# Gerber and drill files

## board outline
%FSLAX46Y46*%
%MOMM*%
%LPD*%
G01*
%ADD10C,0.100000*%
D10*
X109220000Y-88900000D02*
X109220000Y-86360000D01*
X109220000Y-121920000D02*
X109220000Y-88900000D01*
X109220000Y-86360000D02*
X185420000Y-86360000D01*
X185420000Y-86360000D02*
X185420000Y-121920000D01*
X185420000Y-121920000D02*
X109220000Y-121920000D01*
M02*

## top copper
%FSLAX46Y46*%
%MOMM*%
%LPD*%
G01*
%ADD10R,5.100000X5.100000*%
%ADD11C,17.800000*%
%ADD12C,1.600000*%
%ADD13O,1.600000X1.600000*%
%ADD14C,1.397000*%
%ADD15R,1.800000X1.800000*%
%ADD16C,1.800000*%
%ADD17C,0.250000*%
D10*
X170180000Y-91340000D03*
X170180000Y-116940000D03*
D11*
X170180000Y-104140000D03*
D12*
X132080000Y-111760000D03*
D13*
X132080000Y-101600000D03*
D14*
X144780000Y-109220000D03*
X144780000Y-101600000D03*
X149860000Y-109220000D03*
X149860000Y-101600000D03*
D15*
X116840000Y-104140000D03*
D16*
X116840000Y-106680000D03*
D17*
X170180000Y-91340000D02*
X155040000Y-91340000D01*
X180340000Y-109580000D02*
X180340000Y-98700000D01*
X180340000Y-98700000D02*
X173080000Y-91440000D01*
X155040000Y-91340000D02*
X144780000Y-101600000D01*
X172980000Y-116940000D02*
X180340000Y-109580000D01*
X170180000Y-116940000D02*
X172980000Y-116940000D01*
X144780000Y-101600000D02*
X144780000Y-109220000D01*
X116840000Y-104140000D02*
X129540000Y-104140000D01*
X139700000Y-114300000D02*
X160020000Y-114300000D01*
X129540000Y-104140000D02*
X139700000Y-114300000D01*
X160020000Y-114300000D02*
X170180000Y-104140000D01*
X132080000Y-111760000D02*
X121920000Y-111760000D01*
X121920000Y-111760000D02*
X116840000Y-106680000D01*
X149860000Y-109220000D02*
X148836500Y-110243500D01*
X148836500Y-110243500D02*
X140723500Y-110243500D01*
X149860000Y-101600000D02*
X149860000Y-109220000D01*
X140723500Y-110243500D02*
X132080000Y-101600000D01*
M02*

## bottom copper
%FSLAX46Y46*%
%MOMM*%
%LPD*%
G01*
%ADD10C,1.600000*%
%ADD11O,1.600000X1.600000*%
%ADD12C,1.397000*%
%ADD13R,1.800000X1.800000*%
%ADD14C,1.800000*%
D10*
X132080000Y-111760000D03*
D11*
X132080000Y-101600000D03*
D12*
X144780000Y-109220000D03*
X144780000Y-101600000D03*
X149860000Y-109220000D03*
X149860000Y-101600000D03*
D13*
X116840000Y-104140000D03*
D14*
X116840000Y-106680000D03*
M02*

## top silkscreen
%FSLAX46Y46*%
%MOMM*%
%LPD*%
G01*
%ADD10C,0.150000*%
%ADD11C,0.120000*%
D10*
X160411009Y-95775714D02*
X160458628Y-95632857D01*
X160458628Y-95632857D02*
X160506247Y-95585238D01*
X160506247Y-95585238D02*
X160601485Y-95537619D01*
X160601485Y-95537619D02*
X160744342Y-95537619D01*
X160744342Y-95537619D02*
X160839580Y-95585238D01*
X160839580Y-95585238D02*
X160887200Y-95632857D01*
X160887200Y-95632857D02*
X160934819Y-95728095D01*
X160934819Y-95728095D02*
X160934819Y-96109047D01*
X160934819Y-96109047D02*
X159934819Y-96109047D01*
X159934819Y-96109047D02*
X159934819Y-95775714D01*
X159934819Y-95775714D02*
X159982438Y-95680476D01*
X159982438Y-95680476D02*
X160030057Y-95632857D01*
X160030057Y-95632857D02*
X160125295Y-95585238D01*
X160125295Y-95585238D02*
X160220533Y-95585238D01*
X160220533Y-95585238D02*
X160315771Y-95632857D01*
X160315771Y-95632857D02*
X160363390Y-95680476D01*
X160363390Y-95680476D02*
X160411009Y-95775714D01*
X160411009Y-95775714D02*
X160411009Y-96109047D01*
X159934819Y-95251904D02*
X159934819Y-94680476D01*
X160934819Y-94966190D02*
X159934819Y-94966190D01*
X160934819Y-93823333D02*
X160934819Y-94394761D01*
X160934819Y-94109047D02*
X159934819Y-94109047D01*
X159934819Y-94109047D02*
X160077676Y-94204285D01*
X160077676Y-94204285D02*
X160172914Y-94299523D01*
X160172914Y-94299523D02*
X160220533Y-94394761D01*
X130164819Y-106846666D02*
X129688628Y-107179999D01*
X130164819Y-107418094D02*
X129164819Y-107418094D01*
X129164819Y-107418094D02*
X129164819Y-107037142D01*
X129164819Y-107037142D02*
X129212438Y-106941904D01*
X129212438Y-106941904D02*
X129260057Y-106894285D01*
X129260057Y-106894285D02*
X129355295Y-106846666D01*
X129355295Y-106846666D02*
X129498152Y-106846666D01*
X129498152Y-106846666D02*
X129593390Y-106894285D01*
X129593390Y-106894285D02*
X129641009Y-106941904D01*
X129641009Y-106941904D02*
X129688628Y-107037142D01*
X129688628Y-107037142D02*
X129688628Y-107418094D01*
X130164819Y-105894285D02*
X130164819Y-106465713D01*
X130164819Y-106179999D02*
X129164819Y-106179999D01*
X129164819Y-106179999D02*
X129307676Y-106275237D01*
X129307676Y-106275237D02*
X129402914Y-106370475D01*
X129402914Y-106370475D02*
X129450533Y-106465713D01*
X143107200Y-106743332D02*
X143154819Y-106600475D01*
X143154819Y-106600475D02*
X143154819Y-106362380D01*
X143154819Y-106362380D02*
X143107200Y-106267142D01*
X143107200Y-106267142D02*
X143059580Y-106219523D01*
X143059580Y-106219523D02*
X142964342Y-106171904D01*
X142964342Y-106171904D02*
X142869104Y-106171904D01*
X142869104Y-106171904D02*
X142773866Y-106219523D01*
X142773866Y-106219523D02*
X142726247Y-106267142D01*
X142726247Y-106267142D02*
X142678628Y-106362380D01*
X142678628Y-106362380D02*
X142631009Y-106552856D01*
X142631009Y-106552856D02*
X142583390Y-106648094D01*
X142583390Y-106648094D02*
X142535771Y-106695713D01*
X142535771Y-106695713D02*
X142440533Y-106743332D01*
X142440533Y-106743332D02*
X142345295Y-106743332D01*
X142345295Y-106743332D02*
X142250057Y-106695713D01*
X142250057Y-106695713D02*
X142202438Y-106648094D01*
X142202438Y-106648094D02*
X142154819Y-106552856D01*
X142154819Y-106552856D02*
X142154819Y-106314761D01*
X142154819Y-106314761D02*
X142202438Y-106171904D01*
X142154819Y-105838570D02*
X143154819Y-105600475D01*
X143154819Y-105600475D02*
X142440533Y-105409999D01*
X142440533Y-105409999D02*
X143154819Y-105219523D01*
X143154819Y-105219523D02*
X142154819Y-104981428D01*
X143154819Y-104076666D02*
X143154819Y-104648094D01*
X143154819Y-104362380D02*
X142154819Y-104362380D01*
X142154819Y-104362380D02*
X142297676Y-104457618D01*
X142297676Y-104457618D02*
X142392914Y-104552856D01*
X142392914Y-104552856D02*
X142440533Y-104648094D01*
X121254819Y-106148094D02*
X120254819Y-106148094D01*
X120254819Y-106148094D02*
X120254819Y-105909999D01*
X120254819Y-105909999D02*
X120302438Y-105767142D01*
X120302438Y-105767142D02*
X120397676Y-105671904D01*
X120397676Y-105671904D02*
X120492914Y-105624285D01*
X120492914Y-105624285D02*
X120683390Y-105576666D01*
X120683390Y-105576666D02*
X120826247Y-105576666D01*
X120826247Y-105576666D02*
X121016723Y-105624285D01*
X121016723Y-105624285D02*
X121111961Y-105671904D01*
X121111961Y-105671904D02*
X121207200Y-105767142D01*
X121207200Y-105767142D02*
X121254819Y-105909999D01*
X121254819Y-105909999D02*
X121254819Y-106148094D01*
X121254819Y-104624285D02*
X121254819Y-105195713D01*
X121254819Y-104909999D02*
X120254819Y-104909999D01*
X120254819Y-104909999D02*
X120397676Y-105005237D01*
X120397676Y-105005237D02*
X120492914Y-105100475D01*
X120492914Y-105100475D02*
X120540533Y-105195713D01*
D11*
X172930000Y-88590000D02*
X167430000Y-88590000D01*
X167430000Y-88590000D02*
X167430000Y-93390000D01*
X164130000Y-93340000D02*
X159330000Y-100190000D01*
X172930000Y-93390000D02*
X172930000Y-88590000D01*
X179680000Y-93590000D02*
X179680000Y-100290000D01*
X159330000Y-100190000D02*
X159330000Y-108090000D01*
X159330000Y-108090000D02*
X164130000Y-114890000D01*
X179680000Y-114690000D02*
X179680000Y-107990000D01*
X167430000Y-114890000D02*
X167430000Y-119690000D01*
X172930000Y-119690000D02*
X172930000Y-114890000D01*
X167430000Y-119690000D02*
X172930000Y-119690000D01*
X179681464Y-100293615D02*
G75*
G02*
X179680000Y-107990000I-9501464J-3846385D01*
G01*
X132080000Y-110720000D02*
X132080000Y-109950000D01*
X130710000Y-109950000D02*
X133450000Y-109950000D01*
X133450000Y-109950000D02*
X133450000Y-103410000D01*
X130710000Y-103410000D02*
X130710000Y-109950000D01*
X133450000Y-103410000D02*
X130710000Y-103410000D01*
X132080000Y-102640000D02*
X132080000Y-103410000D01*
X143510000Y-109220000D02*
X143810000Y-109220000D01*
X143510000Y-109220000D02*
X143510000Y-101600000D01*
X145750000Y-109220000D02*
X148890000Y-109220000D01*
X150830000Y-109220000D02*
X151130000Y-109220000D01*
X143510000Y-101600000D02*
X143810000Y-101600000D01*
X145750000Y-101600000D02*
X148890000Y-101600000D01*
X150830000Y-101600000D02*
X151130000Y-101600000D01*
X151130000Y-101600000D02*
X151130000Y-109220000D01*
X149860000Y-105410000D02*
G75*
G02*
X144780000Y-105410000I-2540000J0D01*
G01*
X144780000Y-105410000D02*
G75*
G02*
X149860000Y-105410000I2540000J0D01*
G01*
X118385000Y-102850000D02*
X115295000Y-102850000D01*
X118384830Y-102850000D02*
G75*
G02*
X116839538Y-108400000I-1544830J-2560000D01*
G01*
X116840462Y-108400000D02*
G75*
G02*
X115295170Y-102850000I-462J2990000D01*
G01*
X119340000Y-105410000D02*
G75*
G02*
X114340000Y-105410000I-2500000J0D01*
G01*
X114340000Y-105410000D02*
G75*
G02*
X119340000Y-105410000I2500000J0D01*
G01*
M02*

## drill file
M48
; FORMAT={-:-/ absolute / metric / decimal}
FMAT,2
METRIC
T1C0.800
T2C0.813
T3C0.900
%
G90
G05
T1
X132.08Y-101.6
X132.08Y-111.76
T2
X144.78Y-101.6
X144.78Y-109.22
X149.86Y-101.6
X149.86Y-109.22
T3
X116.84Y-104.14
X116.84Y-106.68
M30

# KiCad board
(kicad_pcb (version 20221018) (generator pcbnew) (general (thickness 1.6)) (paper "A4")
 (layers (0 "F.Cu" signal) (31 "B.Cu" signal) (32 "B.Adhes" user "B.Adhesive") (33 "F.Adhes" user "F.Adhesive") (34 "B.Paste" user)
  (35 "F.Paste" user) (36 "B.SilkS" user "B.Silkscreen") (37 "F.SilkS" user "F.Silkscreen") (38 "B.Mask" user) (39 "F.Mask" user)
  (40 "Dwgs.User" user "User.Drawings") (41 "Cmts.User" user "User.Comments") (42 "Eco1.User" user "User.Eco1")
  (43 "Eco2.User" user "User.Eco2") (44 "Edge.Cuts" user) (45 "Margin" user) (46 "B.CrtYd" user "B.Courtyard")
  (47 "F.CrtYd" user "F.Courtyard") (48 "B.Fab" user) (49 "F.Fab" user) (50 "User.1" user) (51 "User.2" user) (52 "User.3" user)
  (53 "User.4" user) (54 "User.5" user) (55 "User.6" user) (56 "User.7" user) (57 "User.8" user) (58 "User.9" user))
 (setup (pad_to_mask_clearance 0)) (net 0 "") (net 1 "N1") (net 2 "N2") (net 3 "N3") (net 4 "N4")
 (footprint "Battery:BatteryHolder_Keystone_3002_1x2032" (layer "F.Cu") (at 170.18 104.14 -90)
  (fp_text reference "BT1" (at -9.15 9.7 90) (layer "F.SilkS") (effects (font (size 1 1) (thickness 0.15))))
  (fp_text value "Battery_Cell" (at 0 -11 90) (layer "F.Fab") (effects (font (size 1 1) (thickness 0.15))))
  (fp_line (start -15.55 -2.75) (end -15.55 2.75) (stroke (width 0.12) (type solid)) (layer "F.SilkS"))
  (fp_line (start -15.55 2.75) (end -10.75 2.75) (stroke (width 0.12) (type solid)) (layer "F.SilkS"))
  (fp_line (start -10.8 6.05) (end -3.95 10.85) (stroke (width 0.12) (type solid)) (layer "F.SilkS"))
  (fp_line (start -10.75 -2.75) (end -15.55 -2.75) (stroke (width 0.12) (type solid)) (layer "F.SilkS"))
  (fp_line (start -10.55 -9.5) (end -3.85 -9.5) (stroke (width 0.12) (type solid)) (layer "F.SilkS"))
  (fp_line (start -3.95 10.85) (end 3.95 10.85) (stroke (width 0.12) (type solid)) (layer "F.SilkS"))
  (fp_line (start 3.95 10.85) (end 10.75 6.05) (stroke (width 0.12) (type solid)) (layer "F.SilkS"))
  (fp_line (start 10.55 -9.5) (end 3.85 -9.5) (stroke (width 0.12) (type solid)) (layer "F.SilkS"))
  (fp_line (start 10.75 2.75) (end 15.55 2.75) (stroke (width 0.12) (type solid)) (layer "F.SilkS"))
  (fp_line (start 15.55 -2.75) (end 10.75 -2.75) (stroke (width 0.12) (type solid)) (layer "F.SilkS"))
  (fp_line (start 15.55 2.75) (end 15.55 -2.75) (stroke (width 0.12) (type solid)) (layer "F.SilkS"))
  (fp_arc (start -3.846385 -9.501464) (mid 0.00195 -10.250487) (end 3.85 -9.5) (stroke (width 0.12) (type solid)) (layer "F.SilkS"))
  (pad "1" smd rect (at -12.8 0 270) (size 5.1 5.1) (layers "F.Cu" "F.Paste" "F.Mask") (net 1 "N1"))
  (pad "1" smd rect (at 12.8 0 270) (size 5.1 5.1) (layers "F.Cu" "F.Paste" "F.Mask") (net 1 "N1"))
  (pad "2" smd circle (at 0 0 270) (size 17.8 17.8) (layers "F.Cu" "F.Mask") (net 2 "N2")))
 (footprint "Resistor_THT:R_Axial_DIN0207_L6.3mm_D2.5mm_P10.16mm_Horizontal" (layer "F.Cu") (at 132.08 111.76 90)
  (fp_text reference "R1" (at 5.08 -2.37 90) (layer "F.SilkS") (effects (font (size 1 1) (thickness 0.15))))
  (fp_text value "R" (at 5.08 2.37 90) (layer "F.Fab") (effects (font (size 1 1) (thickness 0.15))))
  (fp_line (start 1.04 0) (end 1.81 0) (stroke (width 0.12) (type solid)) (layer "F.SilkS"))
  (fp_line (start 1.81 -1.37) (end 1.81 1.37) (stroke (width 0.12) (type solid)) (layer "F.SilkS"))
  (fp_line (start 1.81 1.37) (end 8.35 1.37) (stroke (width 0.12) (type solid)) (layer "F.SilkS"))
  (fp_line (start 8.35 -1.37) (end 1.81 -1.37) (stroke (width 0.12) (type solid)) (layer "F.SilkS"))
  (fp_line (start 8.35 1.37) (end 8.35 -1.37) (stroke (width 0.12) (type solid)) (layer "F.SilkS"))
  (fp_line (start 9.12 0) (end 8.35 0) (stroke (width 0.12) (type solid)) (layer "F.SilkS"))
  (pad "1" thru_hole circle (at 0 0 90) (size 1.6 1.6) (drill 0.8) (layers "*.Cu" "*.Mask") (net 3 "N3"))
  (pad "2" thru_hole oval (at 10.16 0 90) (size 1.6 1.6) (drill 0.8) (layers "*.Cu" "*.Mask") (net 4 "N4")))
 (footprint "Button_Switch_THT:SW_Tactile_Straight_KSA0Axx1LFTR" (layer "F.Cu") (at 144.78 109.22 90)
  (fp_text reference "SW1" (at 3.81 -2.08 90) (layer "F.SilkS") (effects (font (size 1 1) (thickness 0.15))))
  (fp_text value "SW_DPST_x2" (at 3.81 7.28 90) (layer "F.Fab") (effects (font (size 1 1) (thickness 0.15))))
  (fp_line (start 0 -1.27) (end 0 -0.97) (stroke (width 0.12) (type solid)) (layer "F.SilkS"))
  (fp_line (start 0 -1.27) (end 7.62 -1.27) (stroke (width 0.12) (type solid)) (layer "F.SilkS"))
  (fp_line (start 0 0.97) (end 0 4.11) (stroke (width 0.12) (type solid)) (layer "F.SilkS"))
  (fp_line (start 0 6.05) (end 0 6.35) (stroke (width 0.12) (type solid)) (layer "F.SilkS"))
  (fp_line (start 7.62 -1.27) (end 7.62 -0.97) (stroke (width 0.12) (type solid)) (layer "F.SilkS"))
  (fp_line (start 7.62 0.97) (end 7.62 4.11) (stroke (width 0.12) (type solid)) (layer "F.SilkS"))
  (fp_line (start 7.62 6.05) (end 7.62 6.35) (stroke (width 0.12) (type solid)) (layer "F.SilkS"))
  (fp_line (start 7.62 6.35) (end 0 6.35) (stroke (width 0.12) (type solid)) (layer "F.SilkS"))
  (fp_circle (center 3.81 2.54) (end 3.81 0) (stroke (width 0.12) (type solid)) (fill none) (layer "F.SilkS"))
  (pad "1" thru_hole circle (at 0 0 90) (size 1.397 1.397) (drill 0.8128) (layers "*.Cu" "*.Mask") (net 1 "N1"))
  (pad "1" thru_hole circle (at 7.62 0 90) (size 1.397 1.397) (drill 0.8128) (layers "*.Cu" "*.Mask") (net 1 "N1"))
  (pad "2" thru_hole circle (at 0 5.08 90) (size 1.397 1.397) (drill 0.8128) (layers "*.Cu" "*.Mask") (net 4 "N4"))
  (pad "2" thru_hole circle (at 7.62 5.08 90) (size 1.397 1.397) (drill 0.8128) (layers "*.Cu" "*.Mask") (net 4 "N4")))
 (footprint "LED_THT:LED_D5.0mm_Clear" (layer "F.Cu") (at 116.84 104.14 -90)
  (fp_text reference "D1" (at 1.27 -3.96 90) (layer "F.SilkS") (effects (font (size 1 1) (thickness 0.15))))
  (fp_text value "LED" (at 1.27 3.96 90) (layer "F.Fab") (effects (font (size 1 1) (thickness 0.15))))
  (fp_line (start -1.29 -1.545) (end -1.29 1.545) (stroke (width 0.12) (type solid)) (layer "F.SilkS"))
  (fp_arc (start -1.29 -1.54483) (mid 2.072002 -2.880433) (end 4.26 0.000462) (stroke (width 0.12) (type solid)) (layer "F.SilkS"))
  (fp_arc (start 4.26 -0.000462) (mid 2.072002 2.880433) (end -1.29 1.54483) (stroke (width 0.12) (type solid)) (layer "F.SilkS"))
  (fp_circle (center 1.27 0) (end 3.77 0) (stroke (width 0.12) (type solid)) (fill none) (layer "F.SilkS"))
  (pad "1" thru_hole rect (at 0 0 270) (size 1.8 1.8) (drill 0.9) (layers "*.Cu" "*.Mask") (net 2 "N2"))
  (pad "2" thru_hole circle (at 2.54 0 270) (size 1.8 1.8) (drill 0.9) (layers "*.Cu" "*.Mask") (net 3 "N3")))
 (gr_line (start 109.22 88.9) (end 109.22 86.36) (stroke (width 0.1) (type default)) (layer "Edge.Cuts"))
 (gr_line (start 109.22 121.92) (end 109.22 88.9) (stroke (width 0.1) (type default)) (layer "Edge.Cuts"))
 (gr_line (start 109.22 86.36) (end 185.42 86.36) (stroke (width 0.1) (type default)) (layer "Edge.Cuts"))
 (gr_line (start 185.42 86.36) (end 185.42 121.92) (stroke (width 0.1) (type default)) (layer "Edge.Cuts"))
 (gr_line (start 185.42 121.92) (end 109.22 121.92) (stroke (width 0.1) (type default)) (layer "Edge.Cuts"))
 (segment (start 170.18 91.34) (end 155.04 91.34) (width 0.25) (layer "F.Cu") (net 1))
 (segment (start 180.34 109.58) (end 180.34 98.7) (width 0.25) (layer "F.Cu") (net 1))
 (segment (start 180.34 98.7) (end 173.08 91.44) (width 0.25) (layer "F.Cu") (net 1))
 (segment (start 155.04 91.34) (end 144.78 101.6) (width 0.25) (layer "F.Cu") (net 1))
 (segment (start 172.98 116.94) (end 180.34 109.58) (width 0.25) (layer "F.Cu") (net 1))
 (segment (start 170.18 116.94) (end 172.98 116.94) (width 0.25) (layer "F.Cu") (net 1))
 (segment (start 144.78 101.6) (end 144.78 109.22) (width 0.25) (layer "F.Cu") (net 1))
 (segment (start 116.84 104.14) (end 129.54 104.14) (width 0.25) (layer "F.Cu") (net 2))
 (segment (start 139.7 114.3) (end 160.02 114.3) (width 0.25) (layer "F.Cu") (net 2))
 (segment (start 129.54 104.14) (end 139.7 114.3) (width 0.25) (layer "F.Cu") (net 2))
 (segment (start 160.02 114.3) (end 170.18 104.14) (width 0.25) (layer "F.Cu") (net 2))
 (segment (start 132.08 111.76) (end 121.92 111.76) (width 0.25) (layer "F.Cu") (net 3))
 (segment (start 121.92 111.76) (end 116.84 106.68) (width 0.25) (layer "F.Cu") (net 3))
 (segment (start 149.86 109.22) (end 148.8365 110.2435) (width 0.25) (layer "F.Cu") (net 4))
 (segment (start 148.8365 110.2435) (end 140.7235 110.2435) (width 0.25) (layer "F.Cu") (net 4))
 (segment (start 149.86 101.6) (end 149.86 109.22) (width 0.25) (layer "F.Cu") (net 4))
 (segment (start 140.7235 110.2435) (end 132.08 101.6) (width 0.25) (layer "F.Cu") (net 4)))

